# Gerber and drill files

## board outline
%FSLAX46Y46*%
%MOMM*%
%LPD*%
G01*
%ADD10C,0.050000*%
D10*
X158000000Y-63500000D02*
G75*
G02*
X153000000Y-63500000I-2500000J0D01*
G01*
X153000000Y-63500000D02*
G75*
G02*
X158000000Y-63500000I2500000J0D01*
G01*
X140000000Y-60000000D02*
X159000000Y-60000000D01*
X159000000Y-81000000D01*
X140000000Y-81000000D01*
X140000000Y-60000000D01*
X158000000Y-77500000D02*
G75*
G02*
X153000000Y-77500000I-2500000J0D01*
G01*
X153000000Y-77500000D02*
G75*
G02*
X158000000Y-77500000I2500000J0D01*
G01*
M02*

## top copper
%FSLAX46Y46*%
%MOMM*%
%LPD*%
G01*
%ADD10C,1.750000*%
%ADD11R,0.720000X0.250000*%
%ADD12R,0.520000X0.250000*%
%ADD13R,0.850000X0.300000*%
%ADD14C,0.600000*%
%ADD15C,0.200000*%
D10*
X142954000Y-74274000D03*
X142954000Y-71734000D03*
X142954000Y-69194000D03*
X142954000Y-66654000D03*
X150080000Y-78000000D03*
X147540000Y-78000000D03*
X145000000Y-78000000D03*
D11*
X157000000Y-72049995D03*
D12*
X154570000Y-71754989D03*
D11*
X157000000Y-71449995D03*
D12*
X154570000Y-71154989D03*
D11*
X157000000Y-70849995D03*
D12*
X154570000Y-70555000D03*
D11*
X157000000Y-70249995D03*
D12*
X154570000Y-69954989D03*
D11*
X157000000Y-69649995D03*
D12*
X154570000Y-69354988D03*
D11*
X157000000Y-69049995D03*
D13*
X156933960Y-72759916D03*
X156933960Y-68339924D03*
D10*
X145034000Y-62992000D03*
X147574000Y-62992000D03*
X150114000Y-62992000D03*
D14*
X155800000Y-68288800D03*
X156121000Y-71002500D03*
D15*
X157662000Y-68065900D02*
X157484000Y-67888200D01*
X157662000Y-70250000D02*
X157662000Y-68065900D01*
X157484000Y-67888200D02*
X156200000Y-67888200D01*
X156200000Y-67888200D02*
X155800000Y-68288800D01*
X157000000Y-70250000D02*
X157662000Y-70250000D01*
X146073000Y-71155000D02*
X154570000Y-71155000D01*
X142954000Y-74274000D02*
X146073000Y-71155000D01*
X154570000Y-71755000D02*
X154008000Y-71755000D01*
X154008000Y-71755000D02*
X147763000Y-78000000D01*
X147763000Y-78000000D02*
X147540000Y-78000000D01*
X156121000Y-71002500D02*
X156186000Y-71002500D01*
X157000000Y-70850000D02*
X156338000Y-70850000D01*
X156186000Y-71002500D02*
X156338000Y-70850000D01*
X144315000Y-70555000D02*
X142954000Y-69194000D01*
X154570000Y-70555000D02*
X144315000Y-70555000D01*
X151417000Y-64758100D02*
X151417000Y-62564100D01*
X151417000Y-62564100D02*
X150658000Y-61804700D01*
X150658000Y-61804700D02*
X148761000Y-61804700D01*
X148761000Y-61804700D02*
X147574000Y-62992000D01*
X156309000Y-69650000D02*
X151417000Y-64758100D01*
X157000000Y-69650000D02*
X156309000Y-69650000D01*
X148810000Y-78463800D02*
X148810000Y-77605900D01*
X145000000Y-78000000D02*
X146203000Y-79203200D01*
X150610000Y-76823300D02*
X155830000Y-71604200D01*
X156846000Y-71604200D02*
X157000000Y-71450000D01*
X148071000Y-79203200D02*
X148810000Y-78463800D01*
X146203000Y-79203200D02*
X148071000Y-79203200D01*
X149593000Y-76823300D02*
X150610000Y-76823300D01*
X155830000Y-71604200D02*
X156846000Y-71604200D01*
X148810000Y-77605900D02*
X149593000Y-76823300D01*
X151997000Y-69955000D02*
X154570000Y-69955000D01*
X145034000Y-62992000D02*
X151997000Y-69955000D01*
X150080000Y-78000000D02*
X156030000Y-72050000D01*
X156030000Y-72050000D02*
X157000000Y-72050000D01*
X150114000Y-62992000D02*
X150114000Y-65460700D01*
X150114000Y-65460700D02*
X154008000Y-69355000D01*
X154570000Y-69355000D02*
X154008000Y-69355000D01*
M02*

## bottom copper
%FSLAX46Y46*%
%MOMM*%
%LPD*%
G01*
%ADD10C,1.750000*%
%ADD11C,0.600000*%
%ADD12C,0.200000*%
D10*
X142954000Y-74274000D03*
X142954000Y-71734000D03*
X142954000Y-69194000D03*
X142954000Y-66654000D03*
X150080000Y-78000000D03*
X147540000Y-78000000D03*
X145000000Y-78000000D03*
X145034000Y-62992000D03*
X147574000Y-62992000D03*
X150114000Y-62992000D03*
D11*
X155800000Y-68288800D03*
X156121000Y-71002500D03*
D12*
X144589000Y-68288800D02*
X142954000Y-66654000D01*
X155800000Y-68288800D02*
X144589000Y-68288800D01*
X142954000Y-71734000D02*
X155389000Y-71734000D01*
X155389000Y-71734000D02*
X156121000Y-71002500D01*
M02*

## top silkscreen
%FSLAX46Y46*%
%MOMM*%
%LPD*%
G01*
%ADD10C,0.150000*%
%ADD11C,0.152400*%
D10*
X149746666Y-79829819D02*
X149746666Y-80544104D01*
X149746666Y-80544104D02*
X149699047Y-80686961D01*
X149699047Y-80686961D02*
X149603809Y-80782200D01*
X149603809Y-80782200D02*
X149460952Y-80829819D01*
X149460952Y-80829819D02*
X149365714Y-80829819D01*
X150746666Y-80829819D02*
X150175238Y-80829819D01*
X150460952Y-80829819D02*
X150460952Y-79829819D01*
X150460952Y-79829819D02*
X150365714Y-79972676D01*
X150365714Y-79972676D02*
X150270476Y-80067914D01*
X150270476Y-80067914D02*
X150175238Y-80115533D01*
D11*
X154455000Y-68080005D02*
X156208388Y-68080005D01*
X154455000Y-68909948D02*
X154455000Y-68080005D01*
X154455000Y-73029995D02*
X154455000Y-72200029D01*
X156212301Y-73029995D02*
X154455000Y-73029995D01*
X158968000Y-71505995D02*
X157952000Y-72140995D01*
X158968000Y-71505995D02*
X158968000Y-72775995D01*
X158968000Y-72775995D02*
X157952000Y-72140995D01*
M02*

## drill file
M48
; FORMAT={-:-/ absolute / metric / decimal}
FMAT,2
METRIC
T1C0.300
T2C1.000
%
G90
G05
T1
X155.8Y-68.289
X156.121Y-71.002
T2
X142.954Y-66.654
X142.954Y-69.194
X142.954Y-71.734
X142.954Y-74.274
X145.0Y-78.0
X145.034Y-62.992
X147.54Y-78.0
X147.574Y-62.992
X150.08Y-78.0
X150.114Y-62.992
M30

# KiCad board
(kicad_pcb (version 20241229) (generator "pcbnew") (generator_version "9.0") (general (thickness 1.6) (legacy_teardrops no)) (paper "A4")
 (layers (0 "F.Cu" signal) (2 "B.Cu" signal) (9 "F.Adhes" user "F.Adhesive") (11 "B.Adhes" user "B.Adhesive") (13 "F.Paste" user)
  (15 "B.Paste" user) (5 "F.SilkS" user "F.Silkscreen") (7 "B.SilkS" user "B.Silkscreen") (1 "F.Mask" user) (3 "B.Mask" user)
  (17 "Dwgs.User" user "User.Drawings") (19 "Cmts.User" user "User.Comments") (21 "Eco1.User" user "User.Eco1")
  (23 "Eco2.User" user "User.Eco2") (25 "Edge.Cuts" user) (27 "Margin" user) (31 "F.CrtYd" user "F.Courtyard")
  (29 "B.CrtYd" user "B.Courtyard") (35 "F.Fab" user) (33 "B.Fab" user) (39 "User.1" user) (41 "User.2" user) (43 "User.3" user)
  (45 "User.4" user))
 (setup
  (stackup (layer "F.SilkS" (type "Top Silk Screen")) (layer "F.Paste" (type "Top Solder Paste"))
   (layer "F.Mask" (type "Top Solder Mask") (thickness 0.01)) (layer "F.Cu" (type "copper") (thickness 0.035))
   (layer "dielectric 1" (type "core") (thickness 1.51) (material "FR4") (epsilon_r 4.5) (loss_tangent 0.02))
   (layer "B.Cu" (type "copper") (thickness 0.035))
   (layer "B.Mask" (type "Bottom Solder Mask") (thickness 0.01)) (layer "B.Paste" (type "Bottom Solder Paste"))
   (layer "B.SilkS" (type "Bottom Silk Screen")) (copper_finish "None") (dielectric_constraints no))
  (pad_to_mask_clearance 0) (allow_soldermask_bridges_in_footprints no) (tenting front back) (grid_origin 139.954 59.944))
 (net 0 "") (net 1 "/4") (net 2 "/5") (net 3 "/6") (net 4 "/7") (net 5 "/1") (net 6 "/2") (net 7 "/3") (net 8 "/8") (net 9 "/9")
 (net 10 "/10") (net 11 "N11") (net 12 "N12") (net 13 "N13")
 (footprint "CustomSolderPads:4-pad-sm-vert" (layer "F.Cu") (at 142.954 74.274 180)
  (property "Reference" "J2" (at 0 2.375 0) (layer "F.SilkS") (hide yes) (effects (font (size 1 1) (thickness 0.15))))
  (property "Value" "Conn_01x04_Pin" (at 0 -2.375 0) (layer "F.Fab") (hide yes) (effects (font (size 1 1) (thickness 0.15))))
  (pad "1" thru_hole circle (at 0 0 180) (size 1.75 1.75) (drill 1) (layers "*.Cu" "*.Mask") (remove_unused_layers no) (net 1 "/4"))
  (pad "2" thru_hole circle (at 0 2.54 180) (size 1.75 1.75) (drill 1) (layers "*.Cu" "*.Mask") (remove_unused_layers no) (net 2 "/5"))
  (pad "3" thru_hole circle (at 0 5.08 180) (size 1.75 1.75) (drill 1) (layers "*.Cu" "*.Mask") (remove_unused_layers no) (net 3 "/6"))
  (pad "4" thru_hole circle (at 0 7.62 180) (size 1.75 1.75) (drill 1) (layers "*.Cu" "*.Mask") (remove_unused_layers no) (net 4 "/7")))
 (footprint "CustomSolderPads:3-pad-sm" (layer "F.Cu") (at 150.08 78)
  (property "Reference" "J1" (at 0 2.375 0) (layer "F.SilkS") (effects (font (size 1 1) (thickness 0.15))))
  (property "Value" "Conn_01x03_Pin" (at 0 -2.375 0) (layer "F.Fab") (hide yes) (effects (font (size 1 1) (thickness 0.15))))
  (pad "1" thru_hole circle (at 0 0) (size 1.75 1.75) (drill 1) (layers "*.Cu" "*.Mask") (remove_unused_layers no) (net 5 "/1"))
  (pad "2" thru_hole circle (at -2.54 0) (size 1.75 1.75) (drill 1) (layers "*.Cu" "*.Mask") (remove_unused_layers no) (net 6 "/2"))
  (pad "3" thru_hole circle (at -5.08 0) (size 1.75 1.75) (drill 1) (layers "*.Cu" "*.Mask") (remove_unused_layers no) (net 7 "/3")))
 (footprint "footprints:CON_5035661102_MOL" (layer "F.Cu") (at 155.88 70.555 90)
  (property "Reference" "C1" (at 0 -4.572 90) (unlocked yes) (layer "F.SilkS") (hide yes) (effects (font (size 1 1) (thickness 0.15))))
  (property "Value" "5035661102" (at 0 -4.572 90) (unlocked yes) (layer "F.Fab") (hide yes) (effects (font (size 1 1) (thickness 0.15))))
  (fp_line (start 2.474995 -1.425) (end 2.474995 0.328388) (stroke (width 0.1524) (type solid)) (layer "F.SilkS"))
  (fp_line (start 1.645052 -1.425) (end 2.474995 -1.425) (stroke (width 0.1524) (type solid)) (layer "F.SilkS"))
  (fp_line (start -2.474995 -1.425) (end -1.645029 -1.425) (stroke (width 0.1524) (type solid)) (layer "F.SilkS"))
  (fp_line (start -2.474995 0.332301) (end -2.474995 -1.425) (stroke (width 0.1524) (type solid)) (layer "F.SilkS"))
  (fp_line (start -0.950995 3.088) (end -1.585995 2.072) (stroke (width 0.1524) (type solid)) (layer "F.SilkS"))
  (fp_line (start -0.950995 3.088) (end -2.220995 3.088) (stroke (width 0.1524) (type solid)) (layer "F.SilkS"))
  (fp_line (start -2.220995 3.088) (end -1.585995 2.072) (stroke (width 0.1524) (type solid)) (layer "F.SilkS"))
  (pad "1" smd rect (at -1.494995 1.12 90) (size 0.25 0.72) (layers "F.Cu" "F.Mask" "F.Paste") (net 5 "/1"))
  (pad "2" smd rect (at -1.199989 -1.31 90) (size 0.25 0.52) (layers "F.Cu" "F.Mask" "F.Paste") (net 6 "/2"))
  (pad "3" smd rect (at -0.894995 1.12 90) (size 0.25 0.72) (layers "F.Cu" "F.Mask" "F.Paste") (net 7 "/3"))
  (pad "4" smd rect (at -0.599989 -1.31 90) (size 0.25 0.52) (layers "F.Cu" "F.Mask" "F.Paste") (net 1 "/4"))
  (pad "5" smd rect (at -0.294995 1.12 90) (size 0.25 0.72) (layers "F.Cu" "F.Mask" "F.Paste") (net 2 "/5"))
  (pad "6" smd rect (at 0 -1.31 90) (size 0.25 0.52) (layers "F.Cu" "F.Mask" "F.Paste") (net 3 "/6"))
  (pad "7" smd rect (at 0.305005 1.12 90) (size 0.25 0.72) (layers "F.Cu" "F.Mask" "F.Paste") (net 4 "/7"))
  (pad "8" smd rect (at 0.600011 -1.31 90) (size 0.25 0.52) (layers "F.Cu" "F.Mask" "F.Paste") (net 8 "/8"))
  (pad "9" smd rect (at 0.905005 1.12 90) (size 0.25 0.72) (layers "F.Cu" "F.Mask" "F.Paste") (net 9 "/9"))
  (pad "10" smd rect (at 1.200012 -1.31 90) (size 0.25 0.52) (layers "F.Cu" "F.Mask" "F.Paste") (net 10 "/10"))
  (pad "11" smd rect (at 1.505005 1.12 90) (size 0.25 0.72) (layers "F.Cu" "F.Mask" "F.Paste") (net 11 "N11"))
  (pad "P1" smd rect (at -2.204916 1.05396 90) (size 0.3 0.85) (layers "F.Cu" "F.Mask" "F.Paste") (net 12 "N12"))
  (pad "P2" smd rect (at 2.215076 1.05396 90) (size 0.3 0.85) (layers "F.Cu" "F.Mask" "F.Paste") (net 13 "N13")))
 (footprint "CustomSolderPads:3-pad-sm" (layer "F.Cu") (at 145.034 62.992 180)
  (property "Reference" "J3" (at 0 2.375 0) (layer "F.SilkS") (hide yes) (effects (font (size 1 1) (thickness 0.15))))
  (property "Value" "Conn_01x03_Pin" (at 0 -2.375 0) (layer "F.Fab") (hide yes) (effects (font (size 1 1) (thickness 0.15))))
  (pad "1" thru_hole circle (at 0 0 180) (size 1.75 1.75) (drill 1) (layers "*.Cu" "*.Mask") (remove_unused_layers no) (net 8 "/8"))
  (pad "2" thru_hole circle (at -2.54 0 180) (size 1.75 1.75) (drill 1) (layers "*.Cu" "*.Mask") (remove_unused_layers no) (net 9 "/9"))
  (pad "3" thru_hole circle (at -5.08 0 180) (size 1.75 1.75) (drill 1) (layers "*.Cu" "*.Mask") (remove_unused_layers no) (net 10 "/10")))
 (gr_circle (center 155.5 63.5) (end 158 63.5) (stroke (width 0.05) (type solid)) (fill no) (layer "Edge.Cuts"))
 (gr_rect (start 140 60) (end 159 81) (stroke (width 0.05) (type solid)) (fill no) (layer "Edge.Cuts"))
 (gr_circle (center 155.5 77.5) (end 158 77.5) (stroke (width 0.05) (type solid)) (fill no) (layer "Edge.Cuts"))
 (segment (start 157.662 68.0659) (end 157.484 67.8882) (width 0.2) (layer "F.Cu") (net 4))
 (segment (start 157.662 70.25) (end 157.662 68.0659) (width 0.2) (layer "F.Cu") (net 4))
 (segment (start 157.484 67.8882) (end 156.2 67.8882) (width 0.2) (layer "F.Cu") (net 4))
 (segment (start 156.2 67.8882) (end 155.8 68.2888) (width 0.2) (layer "F.Cu") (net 4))
 (segment (start 157 70.25) (end 157.662 70.25) (width 0.2) (layer "F.Cu") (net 4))
 (via (at 155.8 68.2888) (size 0.6) (drill 0.3) (layers "F.Cu" "B.Cu") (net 4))
 (segment (start 144.589 68.2888) (end 142.954 66.654) (width 0.2) (layer "B.Cu") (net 4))
 (segment (start 155.8 68.2888) (end 144.589 68.2888) (width 0.2) (layer "B.Cu") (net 4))
 (segment (start 146.073 71.155) (end 154.57 71.155) (width 0.2) (layer "F.Cu") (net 1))
 (segment (start 142.954 74.274) (end 146.073 71.155) (width 0.2) (layer "F.Cu") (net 1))
 (segment (start 154.57 71.755) (end 154.008 71.755) (width 0.2) (layer "F.Cu") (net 6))
 (segment (start 154.008 71.755) (end 147.763 78) (width 0.2) (layer "F.Cu") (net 6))
 (segment (start 147.763 78) (end 147.54 78) (width 0.2) (layer "F.Cu") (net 6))
 (segment (start 156.121 71.0025) (end 156.186 71.0025) (width 0.2) (layer "F.Cu") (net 2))
 (segment (start 157 70.85) (end 156.338 70.85) (width 0.2) (layer "F.Cu") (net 2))
 (segment (start 156.186 71.0025) (end 156.338 70.85) (width 0.2) (layer "F.Cu") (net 2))
 (via (at 156.121 71.0025) (size 0.6) (drill 0.3) (layers "F.Cu" "B.Cu") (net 2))
 (segment (start 142.954 71.734) (end 155.389 71.734) (width 0.2) (layer "B.Cu") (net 2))
 (segment (start 155.389 71.734) (end 156.121 71.0025) (width 0.2) (layer "B.Cu") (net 2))
 (segment (start 144.315 70.555) (end 142.954 69.194) (width 0.2) (layer "F.Cu") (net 3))
 (segment (start 154.57 70.555) (end 144.315 70.555) (width 0.2) (layer "F.Cu") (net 3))
 (segment (start 151.417 64.7581) (end 151.417 62.5641) (width 0.2) (layer "F.Cu") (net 9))
 (segment (start 151.417 62.5641) (end 150.658 61.8047) (width 0.2) (layer "F.Cu") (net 9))
 (segment (start 150.658 61.8047) (end 148.761 61.8047) (width 0.2) (layer "F.Cu") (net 9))
 (segment (start 148.761 61.8047) (end 147.574 62.992) (width 0.2) (layer "F.Cu") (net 9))
 (segment (start 156.309 69.65) (end 151.417 64.7581) (width 0.2) (layer "F.Cu") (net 9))
 (segment (start 157 69.65) (end 156.309 69.65) (width 0.2) (layer "F.Cu") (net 9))
 (segment (start 148.81 78.4638) (end 148.81 77.6059) (width 0.2) (layer "F.Cu") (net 7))
 (segment (start 145 78) (end 146.203 79.2032) (width 0.2) (layer "F.Cu") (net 7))
 (segment (start 150.61 76.8233) (end 155.83 71.6042) (width 0.2) (layer "F.Cu") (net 7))
 (segment (start 156.846 71.6042) (end 157 71.45) (width 0.2) (layer "F.Cu") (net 7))
 (segment (start 148.071 79.2032) (end 148.81 78.4638) (width 0.2) (layer "F.Cu") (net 7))
 (segment (start 146.203 79.2032) (end 148.071 79.2032) (width 0.2) (layer "F.Cu") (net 7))
 (segment (start 149.593 76.8233) (end 150.61 76.8233) (width 0.2) (layer "F.Cu") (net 7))
 (segment (start 155.83 71.6042) (end 156.846 71.6042) (width 0.2) (layer "F.Cu") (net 7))
 (segment (start 148.81 77.6059) (end 149.593 76.8233) (width 0.2) (layer "F.Cu") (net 7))
 (segment (start 151.997 69.955) (end 154.57 69.955) (width 0.2) (layer "F.Cu") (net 8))
 (segment (start 145.034 62.992) (end 151.997 69.955) (width 0.2) (layer "F.Cu") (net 8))
 (segment (start 150.08 78) (end 156.03 72.05) (width 0.2) (layer "F.Cu") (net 5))
 (segment (start 156.03 72.05) (end 157 72.05) (width 0.2) (layer "F.Cu") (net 5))
 (segment (start 150.114 62.992) (end 150.114 65.4607) (width 0.2) (layer "F.Cu") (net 10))
 (segment (start 150.114 65.4607) (end 154.008 69.355) (width 0.2) (layer "F.Cu") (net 10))
 (segment (start 154.57 69.355) (end 154.008 69.355) (width 0.2) (layer "F.Cu") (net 10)))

